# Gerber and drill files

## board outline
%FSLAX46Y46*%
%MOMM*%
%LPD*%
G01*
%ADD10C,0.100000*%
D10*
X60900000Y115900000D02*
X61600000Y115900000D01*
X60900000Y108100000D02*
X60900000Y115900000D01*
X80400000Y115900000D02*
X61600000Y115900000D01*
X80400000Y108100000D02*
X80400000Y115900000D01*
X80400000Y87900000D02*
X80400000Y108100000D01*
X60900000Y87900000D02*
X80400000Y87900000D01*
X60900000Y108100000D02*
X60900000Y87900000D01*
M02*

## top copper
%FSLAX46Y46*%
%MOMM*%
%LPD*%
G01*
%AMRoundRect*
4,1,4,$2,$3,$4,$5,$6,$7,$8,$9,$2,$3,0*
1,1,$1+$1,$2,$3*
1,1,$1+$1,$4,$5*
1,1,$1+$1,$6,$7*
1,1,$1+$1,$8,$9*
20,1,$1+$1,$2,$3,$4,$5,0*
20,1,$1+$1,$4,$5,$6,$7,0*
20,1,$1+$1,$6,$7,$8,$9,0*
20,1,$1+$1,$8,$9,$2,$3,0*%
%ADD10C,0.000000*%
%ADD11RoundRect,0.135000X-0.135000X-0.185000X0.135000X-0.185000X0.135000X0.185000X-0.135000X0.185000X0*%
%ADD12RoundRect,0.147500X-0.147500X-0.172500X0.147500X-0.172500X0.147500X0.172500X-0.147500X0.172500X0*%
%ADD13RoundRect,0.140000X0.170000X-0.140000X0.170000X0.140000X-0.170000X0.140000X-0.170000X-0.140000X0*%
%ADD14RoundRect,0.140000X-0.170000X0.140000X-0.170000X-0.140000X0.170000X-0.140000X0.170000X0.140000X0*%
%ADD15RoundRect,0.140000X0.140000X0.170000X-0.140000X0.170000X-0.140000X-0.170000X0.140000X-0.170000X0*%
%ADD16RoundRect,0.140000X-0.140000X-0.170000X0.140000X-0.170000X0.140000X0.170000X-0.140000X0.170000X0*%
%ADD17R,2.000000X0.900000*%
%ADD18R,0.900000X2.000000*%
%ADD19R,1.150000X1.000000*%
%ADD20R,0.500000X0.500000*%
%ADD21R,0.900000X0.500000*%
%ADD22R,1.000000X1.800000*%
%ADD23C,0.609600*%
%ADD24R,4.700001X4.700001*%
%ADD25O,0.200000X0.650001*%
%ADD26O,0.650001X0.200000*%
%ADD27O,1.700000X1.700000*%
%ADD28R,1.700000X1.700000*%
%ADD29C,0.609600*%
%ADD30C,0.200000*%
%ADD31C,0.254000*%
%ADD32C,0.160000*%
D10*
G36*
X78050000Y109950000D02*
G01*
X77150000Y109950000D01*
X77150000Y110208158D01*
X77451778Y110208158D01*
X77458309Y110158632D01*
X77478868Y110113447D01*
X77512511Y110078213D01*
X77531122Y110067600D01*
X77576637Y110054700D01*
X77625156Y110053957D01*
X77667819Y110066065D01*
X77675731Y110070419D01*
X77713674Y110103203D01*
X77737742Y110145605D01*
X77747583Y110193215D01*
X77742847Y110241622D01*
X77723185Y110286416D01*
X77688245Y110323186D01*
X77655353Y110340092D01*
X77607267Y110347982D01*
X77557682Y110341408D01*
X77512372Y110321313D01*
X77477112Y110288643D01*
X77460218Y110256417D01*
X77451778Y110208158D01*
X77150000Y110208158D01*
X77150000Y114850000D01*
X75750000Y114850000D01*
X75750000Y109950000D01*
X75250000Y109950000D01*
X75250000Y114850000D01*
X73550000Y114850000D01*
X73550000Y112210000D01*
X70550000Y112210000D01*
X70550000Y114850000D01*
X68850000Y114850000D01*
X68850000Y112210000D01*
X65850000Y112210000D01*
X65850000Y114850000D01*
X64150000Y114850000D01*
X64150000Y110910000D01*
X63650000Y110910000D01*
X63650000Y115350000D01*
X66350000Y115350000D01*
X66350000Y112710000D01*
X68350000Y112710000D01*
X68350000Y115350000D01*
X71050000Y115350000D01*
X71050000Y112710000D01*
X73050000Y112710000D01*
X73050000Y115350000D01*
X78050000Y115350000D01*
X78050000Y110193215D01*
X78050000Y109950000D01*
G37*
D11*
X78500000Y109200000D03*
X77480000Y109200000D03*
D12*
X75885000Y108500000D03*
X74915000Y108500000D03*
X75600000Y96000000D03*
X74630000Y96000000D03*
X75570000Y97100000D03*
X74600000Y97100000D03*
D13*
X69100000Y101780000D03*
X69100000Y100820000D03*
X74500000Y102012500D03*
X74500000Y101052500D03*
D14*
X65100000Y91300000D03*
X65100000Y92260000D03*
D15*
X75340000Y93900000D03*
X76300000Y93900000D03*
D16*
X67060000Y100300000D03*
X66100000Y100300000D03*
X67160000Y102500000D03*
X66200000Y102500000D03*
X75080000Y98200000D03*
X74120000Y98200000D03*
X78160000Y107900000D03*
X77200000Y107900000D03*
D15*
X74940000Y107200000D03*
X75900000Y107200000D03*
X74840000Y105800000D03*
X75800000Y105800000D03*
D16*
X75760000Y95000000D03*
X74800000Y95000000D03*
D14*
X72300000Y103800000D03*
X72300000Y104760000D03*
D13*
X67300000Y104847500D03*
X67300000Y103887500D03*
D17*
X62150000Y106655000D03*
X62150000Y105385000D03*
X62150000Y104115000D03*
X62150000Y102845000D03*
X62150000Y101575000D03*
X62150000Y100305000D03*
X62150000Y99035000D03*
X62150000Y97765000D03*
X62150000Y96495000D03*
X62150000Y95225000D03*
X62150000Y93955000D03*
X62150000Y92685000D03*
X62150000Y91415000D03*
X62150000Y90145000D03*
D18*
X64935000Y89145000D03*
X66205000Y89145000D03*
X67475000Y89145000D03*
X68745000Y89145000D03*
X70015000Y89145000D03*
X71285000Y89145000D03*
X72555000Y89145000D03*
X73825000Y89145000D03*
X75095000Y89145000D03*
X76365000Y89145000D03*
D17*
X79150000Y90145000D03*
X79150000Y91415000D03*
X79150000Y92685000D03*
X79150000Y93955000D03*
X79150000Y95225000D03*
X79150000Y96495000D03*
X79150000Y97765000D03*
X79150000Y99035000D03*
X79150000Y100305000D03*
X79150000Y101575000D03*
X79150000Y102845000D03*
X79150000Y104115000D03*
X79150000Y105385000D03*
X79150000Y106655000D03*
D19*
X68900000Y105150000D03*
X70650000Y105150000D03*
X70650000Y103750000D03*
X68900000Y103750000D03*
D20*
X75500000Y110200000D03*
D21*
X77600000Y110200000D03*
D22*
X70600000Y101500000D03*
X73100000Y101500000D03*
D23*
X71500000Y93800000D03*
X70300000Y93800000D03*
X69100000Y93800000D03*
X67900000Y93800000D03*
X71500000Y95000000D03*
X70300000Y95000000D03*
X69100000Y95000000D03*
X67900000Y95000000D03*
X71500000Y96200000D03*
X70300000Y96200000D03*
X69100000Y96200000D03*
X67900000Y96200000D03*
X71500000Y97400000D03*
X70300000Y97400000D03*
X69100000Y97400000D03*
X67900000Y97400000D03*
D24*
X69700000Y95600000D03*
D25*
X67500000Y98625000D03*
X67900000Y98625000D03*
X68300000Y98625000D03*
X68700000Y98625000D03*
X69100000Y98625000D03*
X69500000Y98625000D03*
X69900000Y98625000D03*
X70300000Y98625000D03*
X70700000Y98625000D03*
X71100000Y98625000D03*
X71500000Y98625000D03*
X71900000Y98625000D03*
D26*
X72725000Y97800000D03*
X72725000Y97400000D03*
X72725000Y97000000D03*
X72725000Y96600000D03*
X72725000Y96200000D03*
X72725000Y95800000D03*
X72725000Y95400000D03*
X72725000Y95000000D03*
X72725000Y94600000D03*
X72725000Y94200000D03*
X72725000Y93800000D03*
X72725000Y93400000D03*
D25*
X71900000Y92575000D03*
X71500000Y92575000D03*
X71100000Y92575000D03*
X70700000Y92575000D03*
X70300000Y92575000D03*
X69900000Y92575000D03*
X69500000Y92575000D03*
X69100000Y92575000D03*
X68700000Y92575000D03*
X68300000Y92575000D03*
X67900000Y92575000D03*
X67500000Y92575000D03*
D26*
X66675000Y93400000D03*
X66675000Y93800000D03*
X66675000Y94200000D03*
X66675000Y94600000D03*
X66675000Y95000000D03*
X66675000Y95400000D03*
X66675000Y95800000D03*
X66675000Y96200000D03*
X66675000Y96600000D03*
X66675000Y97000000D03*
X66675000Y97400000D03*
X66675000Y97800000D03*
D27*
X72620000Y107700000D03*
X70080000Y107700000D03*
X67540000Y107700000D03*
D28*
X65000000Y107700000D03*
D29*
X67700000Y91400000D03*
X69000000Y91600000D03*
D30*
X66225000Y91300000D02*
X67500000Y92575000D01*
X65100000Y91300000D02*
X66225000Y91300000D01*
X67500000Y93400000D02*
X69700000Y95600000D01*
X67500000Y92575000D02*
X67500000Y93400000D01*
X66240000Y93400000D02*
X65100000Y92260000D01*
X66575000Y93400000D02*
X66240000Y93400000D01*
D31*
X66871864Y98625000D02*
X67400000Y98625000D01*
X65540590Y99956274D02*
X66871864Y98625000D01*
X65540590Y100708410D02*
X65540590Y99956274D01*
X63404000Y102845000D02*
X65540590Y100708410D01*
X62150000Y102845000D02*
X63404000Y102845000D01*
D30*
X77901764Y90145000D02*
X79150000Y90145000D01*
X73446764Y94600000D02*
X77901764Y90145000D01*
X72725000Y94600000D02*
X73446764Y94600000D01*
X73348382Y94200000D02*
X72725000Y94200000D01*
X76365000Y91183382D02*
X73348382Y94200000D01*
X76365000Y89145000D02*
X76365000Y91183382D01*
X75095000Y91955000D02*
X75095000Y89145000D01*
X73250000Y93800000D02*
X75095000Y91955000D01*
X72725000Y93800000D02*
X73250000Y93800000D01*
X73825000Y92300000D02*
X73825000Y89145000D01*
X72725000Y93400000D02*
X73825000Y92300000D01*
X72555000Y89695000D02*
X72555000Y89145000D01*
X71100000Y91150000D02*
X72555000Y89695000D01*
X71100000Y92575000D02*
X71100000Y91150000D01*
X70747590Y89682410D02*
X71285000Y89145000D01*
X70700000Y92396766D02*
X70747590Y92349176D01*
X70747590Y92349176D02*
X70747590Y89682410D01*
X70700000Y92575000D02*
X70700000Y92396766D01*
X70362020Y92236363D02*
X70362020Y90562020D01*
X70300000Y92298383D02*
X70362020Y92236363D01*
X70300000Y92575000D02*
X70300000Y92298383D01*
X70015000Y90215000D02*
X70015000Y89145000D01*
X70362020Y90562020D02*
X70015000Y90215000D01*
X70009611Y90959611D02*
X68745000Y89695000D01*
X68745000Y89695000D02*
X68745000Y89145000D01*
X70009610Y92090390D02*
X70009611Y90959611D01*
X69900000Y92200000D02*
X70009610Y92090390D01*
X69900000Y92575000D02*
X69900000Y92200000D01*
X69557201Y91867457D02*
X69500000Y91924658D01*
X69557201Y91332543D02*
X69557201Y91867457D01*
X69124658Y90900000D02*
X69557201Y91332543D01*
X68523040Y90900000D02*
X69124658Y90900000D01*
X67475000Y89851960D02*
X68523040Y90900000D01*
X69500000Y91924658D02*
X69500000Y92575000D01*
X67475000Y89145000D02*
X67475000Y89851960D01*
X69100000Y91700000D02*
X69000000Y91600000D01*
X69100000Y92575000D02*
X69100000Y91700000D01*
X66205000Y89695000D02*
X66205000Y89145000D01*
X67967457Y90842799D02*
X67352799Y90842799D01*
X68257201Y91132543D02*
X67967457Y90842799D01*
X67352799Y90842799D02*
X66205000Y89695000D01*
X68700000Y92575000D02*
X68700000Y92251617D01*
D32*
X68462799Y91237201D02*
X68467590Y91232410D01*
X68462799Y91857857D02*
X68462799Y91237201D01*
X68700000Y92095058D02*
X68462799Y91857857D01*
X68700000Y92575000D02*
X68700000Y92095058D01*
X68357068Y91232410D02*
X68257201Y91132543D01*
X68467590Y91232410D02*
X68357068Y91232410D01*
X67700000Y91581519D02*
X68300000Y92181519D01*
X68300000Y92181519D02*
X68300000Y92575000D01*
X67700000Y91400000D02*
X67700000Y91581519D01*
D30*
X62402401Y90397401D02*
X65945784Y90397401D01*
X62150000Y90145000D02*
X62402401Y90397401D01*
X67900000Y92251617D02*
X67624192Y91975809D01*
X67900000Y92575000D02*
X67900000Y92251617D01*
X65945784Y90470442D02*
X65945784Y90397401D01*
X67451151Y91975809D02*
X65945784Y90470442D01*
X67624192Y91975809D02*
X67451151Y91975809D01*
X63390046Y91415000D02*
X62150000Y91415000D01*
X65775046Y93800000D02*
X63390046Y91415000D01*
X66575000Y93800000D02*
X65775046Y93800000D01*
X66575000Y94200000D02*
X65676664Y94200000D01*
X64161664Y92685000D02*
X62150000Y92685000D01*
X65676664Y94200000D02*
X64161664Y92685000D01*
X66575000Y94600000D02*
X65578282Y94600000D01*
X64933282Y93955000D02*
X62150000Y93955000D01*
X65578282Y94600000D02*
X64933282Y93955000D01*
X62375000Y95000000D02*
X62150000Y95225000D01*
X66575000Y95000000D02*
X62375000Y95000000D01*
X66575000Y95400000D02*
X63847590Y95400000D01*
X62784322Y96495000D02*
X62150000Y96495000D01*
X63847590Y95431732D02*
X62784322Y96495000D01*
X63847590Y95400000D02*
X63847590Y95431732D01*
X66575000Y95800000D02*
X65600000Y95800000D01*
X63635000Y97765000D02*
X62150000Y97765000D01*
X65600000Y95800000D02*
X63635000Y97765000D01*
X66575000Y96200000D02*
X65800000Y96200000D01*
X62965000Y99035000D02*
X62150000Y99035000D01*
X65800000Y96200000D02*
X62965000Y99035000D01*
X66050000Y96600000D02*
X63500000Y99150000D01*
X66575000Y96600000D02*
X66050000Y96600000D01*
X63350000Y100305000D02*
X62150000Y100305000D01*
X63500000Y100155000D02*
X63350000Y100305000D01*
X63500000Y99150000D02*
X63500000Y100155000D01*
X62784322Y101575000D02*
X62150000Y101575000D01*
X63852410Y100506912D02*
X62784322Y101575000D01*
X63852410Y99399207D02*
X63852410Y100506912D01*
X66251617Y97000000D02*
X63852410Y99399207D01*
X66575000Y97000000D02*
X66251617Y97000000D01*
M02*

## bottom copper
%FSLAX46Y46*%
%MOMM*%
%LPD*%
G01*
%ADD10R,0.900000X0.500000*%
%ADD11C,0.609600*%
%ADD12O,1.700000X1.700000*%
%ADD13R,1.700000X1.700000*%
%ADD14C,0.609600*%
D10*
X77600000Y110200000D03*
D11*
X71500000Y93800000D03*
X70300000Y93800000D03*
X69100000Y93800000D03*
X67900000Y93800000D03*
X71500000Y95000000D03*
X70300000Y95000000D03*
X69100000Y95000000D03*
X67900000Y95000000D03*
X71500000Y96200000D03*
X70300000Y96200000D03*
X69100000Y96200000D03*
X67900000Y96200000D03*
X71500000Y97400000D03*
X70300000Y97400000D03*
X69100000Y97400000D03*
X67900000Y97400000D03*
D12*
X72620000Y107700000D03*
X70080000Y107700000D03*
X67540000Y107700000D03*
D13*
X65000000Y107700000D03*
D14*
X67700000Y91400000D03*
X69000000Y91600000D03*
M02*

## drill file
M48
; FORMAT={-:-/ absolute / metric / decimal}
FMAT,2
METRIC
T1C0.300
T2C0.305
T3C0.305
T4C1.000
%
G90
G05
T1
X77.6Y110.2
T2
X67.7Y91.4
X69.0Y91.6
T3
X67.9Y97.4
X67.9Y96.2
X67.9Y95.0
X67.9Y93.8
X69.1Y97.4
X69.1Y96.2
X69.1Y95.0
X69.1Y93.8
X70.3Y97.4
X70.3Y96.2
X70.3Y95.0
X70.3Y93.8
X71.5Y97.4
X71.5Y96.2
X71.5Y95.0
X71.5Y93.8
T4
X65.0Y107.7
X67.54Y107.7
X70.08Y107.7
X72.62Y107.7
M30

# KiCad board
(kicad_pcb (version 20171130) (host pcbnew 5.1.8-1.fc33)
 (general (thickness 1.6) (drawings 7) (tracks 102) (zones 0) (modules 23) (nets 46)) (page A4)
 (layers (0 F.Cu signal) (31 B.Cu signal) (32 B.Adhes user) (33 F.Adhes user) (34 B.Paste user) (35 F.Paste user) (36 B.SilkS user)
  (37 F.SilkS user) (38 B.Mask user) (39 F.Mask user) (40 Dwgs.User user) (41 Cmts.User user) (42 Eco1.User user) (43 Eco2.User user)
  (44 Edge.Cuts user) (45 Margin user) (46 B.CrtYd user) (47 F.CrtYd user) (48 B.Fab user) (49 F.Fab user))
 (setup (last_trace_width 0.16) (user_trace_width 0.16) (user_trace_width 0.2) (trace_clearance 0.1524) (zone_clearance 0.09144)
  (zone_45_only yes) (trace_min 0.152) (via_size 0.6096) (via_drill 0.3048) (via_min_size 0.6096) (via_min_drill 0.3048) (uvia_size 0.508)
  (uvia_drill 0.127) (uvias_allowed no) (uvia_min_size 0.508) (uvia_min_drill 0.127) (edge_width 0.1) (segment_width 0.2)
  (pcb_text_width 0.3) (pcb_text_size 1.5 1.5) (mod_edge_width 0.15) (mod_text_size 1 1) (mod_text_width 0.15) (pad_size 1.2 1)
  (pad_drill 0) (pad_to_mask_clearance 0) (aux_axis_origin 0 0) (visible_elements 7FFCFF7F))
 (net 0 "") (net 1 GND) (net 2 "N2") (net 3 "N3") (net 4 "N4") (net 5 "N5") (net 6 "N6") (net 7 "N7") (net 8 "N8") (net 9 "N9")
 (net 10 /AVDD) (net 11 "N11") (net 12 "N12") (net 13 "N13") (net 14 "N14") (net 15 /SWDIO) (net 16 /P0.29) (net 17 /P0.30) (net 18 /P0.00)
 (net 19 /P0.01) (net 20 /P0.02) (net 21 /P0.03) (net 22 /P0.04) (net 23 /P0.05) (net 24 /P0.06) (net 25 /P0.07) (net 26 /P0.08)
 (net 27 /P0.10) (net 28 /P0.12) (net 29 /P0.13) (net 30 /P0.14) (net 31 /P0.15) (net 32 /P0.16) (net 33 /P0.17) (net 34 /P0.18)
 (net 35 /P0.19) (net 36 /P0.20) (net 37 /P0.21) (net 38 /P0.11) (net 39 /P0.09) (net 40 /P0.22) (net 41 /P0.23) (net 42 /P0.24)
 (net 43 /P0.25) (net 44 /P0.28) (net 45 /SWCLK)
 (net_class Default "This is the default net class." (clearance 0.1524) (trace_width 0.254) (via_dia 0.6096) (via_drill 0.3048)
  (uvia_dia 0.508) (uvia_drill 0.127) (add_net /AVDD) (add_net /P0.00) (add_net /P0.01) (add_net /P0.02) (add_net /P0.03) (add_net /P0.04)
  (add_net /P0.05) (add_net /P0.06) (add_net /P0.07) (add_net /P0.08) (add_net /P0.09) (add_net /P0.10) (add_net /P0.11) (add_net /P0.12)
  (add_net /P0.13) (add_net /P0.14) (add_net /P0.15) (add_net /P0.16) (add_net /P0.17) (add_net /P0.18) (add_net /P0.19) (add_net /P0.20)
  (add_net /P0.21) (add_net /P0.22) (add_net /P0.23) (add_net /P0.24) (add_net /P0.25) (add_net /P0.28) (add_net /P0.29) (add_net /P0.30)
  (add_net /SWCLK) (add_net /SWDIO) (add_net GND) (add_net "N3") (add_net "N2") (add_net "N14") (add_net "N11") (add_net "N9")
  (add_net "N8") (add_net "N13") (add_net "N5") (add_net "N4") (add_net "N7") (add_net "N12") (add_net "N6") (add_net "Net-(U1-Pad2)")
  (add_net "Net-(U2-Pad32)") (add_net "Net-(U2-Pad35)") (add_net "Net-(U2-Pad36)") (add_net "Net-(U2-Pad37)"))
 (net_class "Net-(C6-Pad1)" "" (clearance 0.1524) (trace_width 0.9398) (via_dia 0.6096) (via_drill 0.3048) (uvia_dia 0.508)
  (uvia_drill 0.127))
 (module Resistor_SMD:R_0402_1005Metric (layer F.Cu) (at 77.99 -109.2)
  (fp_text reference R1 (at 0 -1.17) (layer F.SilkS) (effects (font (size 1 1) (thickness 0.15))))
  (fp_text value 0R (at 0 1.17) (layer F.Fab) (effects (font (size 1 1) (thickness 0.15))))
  (pad 2 smd roundrect (at 0.51 0) (size 0.54 0.64) (layers F.Cu F.Paste F.Mask) (roundrect_rratio 0.25) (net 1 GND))
  (pad 1 smd roundrect (at -0.51 0) (size 0.54 0.64) (layers F.Cu F.Paste F.Mask) (roundrect_rratio 0.25) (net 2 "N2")))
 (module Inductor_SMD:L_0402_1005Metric (layer F.Cu) (at 75.4 -108.5)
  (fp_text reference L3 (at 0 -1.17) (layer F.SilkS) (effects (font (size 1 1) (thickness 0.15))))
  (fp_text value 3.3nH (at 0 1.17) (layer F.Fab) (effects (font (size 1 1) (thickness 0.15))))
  (pad 2 smd roundrect (at 0.485 0) (size 0.59 0.64) (layers F.Cu F.Paste F.Mask) (roundrect_rratio 0.25) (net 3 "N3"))
  (pad 1 smd roundrect (at -0.485 0) (size 0.59 0.64) (layers F.Cu F.Paste F.Mask) (roundrect_rratio 0.25) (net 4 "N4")))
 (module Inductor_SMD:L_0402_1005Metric (layer F.Cu) (at 75.115 -96)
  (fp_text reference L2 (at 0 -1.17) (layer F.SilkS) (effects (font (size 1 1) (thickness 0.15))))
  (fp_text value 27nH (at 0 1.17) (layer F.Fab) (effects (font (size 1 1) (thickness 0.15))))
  (pad 2 smd roundrect (at 0.485 0) (size 0.59 0.64) (layers F.Cu F.Paste F.Mask) (roundrect_rratio 0.25) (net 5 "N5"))
  (pad 1 smd roundrect (at -0.485 0) (size 0.59 0.64) (layers F.Cu F.Paste F.Mask) (roundrect_rratio 0.25) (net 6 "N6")))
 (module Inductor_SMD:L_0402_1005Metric (layer F.Cu) (at 75.085 -97.1)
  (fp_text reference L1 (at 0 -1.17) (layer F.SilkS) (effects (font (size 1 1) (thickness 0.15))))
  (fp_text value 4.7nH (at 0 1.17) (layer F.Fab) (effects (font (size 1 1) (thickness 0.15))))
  (pad 2 smd roundrect (at 0.485 0) (size 0.59 0.64) (layers F.Cu F.Paste F.Mask) (roundrect_rratio 0.25) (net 6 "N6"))
  (pad 1 smd roundrect (at -0.485 0) (size 0.59 0.64) (layers F.Cu F.Paste F.Mask) (roundrect_rratio 0.25) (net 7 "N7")))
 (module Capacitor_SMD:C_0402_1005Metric (layer F.Cu) (at 69.1 -101.3 90)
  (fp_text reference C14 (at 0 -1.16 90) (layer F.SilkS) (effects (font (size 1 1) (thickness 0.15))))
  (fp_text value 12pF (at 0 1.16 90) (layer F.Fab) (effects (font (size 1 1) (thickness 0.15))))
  (pad 2 smd roundrect (at 0.48 0 90) (size 0.56 0.62) (layers F.Cu F.Paste F.Mask) (roundrect_rratio 0.25) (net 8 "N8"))
  (pad 1 smd roundrect (at -0.48 0 90) (size 0.56 0.62) (layers F.Cu F.Paste F.Mask) (roundrect_rratio 0.25) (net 1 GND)))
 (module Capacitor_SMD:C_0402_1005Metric (layer F.Cu) (at 74.5 -101.5325 90)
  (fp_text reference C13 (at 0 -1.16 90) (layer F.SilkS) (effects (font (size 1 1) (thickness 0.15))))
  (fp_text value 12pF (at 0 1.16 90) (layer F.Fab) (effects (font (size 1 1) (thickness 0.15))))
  (pad 2 smd roundrect (at 0.48 0 90) (size 0.56 0.62) (layers F.Cu F.Paste F.Mask) (roundrect_rratio 0.25) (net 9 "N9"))
  (pad 1 smd roundrect (at -0.48 0 90) (size 0.56 0.62) (layers F.Cu F.Paste F.Mask) (roundrect_rratio 0.25) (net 1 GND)))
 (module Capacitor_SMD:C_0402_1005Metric (layer F.Cu) (at 65.1 -91.78 270)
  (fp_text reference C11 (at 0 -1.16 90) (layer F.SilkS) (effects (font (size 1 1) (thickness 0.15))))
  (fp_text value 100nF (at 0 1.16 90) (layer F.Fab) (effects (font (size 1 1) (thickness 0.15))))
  (pad 2 smd roundrect (at 0.48 0 270) (size 0.56 0.62) (layers F.Cu F.Paste F.Mask) (roundrect_rratio 0.25) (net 1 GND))
  (pad 1 smd roundrect (at -0.48 0 270) (size 0.56 0.62) (layers F.Cu F.Paste F.Mask) (roundrect_rratio 0.25) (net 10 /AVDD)))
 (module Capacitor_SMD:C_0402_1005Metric (layer F.Cu) (at 75.82 -93.9 180)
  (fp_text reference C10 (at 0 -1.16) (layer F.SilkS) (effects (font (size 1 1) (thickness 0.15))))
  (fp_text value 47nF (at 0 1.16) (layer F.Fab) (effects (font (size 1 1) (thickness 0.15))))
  (pad 2 smd roundrect (at 0.48 0 180) (size 0.56 0.62) (layers F.Cu F.Paste F.Mask) (roundrect_rratio 0.25) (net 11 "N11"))
  (pad 1 smd roundrect (at -0.48 0 180) (size 0.56 0.62) (layers F.Cu F.Paste F.Mask) (roundrect_rratio 0.25) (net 1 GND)))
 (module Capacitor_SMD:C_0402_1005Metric (layer F.Cu) (at 66.58 -100.3)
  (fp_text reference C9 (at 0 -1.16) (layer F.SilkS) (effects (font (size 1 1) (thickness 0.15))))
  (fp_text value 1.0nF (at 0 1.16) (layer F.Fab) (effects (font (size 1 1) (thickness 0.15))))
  (pad 2 smd roundrect (at 0.48 0) (size 0.56 0.62) (layers F.Cu F.Paste F.Mask) (roundrect_rratio 0.25) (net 1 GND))
  (pad 1 smd roundrect (at -0.48 0) (size 0.56 0.62) (layers F.Cu F.Paste F.Mask) (roundrect_rratio 0.25) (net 10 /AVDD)))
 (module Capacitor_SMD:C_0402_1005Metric (layer F.Cu) (at 66.68 -102.5)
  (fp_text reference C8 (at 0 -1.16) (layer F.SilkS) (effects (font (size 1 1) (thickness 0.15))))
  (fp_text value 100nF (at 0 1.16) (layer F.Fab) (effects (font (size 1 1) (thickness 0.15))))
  (pad 2 smd roundrect (at 0.48 0) (size 0.56 0.62) (layers F.Cu F.Paste F.Mask) (roundrect_rratio 0.25) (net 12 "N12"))
  (pad 1 smd roundrect (at -0.48 0) (size 0.56 0.62) (layers F.Cu F.Paste F.Mask) (roundrect_rratio 0.25) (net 1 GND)))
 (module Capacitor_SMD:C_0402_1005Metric (layer F.Cu) (at 74.6 -98.2)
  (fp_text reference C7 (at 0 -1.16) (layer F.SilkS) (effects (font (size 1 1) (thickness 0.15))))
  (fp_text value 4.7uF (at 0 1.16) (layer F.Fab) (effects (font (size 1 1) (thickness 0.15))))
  (pad 2 smd roundrect (at 0.48 0) (size 0.56 0.62) (layers F.Cu F.Paste F.Mask) (roundrect_rratio 0.25) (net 1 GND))
  (pad 1 smd roundrect (at -0.48 0) (size 0.56 0.62) (layers F.Cu F.Paste F.Mask) (roundrect_rratio 0.25) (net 10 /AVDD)))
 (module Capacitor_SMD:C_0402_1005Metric (layer F.Cu) (at 77.68 -107.9)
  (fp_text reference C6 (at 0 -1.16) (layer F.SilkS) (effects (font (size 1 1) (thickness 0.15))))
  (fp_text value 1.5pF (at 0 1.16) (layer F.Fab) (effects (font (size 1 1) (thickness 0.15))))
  (pad 2 smd roundrect (at 0.48 0) (size 0.56 0.62) (layers F.Cu F.Paste F.Mask) (roundrect_rratio 0.25) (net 1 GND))
  (pad 1 smd roundrect (at -0.48 0) (size 0.56 0.62) (layers F.Cu F.Paste F.Mask) (roundrect_rratio 0.25) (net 3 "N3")))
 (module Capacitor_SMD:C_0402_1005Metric (layer F.Cu) (at 75.42 -107.2 180)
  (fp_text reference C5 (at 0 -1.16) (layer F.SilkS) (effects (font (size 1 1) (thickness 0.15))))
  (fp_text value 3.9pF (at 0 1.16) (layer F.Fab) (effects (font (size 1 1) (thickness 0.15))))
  (pad 2 smd roundrect (at 0.48 0 180) (size 0.56 0.62) (layers F.Cu F.Paste F.Mask) (roundrect_rratio 0.25) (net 7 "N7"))
  (pad 1 smd roundrect (at -0.48 0 180) (size 0.56 0.62) (layers F.Cu F.Paste F.Mask) (roundrect_rratio 0.25) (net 4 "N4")))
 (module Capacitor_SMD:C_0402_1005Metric (layer F.Cu) (at 75.32 -105.8 180)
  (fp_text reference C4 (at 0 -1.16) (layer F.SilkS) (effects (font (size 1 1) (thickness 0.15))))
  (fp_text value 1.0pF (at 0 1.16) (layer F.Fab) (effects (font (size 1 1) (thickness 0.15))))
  (pad 2 smd roundrect (at 0.48 0 180) (size 0.56 0.62) (layers F.Cu F.Paste F.Mask) (roundrect_rratio 0.25) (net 1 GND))
  (pad 1 smd roundrect (at -0.48 0 180) (size 0.56 0.62) (layers F.Cu F.Paste F.Mask) (roundrect_rratio 0.25) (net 4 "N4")))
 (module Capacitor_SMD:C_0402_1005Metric (layer F.Cu) (at 75.28 -95)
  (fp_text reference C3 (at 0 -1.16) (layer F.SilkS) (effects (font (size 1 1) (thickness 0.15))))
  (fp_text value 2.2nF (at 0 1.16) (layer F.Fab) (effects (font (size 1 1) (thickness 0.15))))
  (pad 2 smd roundrect (at 0.48 0) (size 0.56 0.62) (layers F.Cu F.Paste F.Mask) (roundrect_rratio 0.25) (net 1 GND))
  (pad 1 smd roundrect (at -0.48 0) (size 0.56 0.62) (layers F.Cu F.Paste F.Mask) (roundrect_rratio 0.25) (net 5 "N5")))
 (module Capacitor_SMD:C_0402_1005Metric (layer F.Cu) (at 72.3 -104.28 270)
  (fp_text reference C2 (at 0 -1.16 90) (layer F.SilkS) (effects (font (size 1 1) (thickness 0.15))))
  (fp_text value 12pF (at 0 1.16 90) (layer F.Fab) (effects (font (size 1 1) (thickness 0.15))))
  (pad 2 smd roundrect (at 0.48 0 270) (size 0.56 0.62) (layers F.Cu F.Paste F.Mask) (roundrect_rratio 0.25) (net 1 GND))
  (pad 1 smd roundrect (at -0.48 0 270) (size 0.56 0.62) (layers F.Cu F.Paste F.Mask) (roundrect_rratio 0.25) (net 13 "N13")))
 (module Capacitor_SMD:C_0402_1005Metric (layer F.Cu) (at 67.3 -104.3675 90)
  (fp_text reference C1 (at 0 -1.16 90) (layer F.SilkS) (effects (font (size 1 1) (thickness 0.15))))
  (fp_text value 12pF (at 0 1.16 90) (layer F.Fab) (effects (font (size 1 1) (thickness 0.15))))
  (pad 2 smd roundrect (at 0.48 0 90) (size 0.56 0.62) (layers F.Cu F.Paste F.Mask) (roundrect_rratio 0.25) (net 1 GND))
  (pad 1 smd roundrect (at -0.48 0 90) (size 0.56 0.62) (layers F.Cu F.Paste F.Mask) (roundrect_rratio 0.25) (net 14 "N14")))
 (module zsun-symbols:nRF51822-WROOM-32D (layer F.Cu) (at 70.65 -98.4)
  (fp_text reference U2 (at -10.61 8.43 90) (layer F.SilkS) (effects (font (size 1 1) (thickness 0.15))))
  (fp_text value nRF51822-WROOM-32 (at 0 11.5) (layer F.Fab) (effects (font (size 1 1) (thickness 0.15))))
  (pad 1 smd rect (at -8.5 -8.255) (size 2 0.9) (layers F.Cu F.Paste F.Mask) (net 1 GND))
  (pad 2 smd rect (at -8.5 -6.985) (size 2 0.9) (layers F.Cu F.Paste F.Mask) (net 10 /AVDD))
  (pad 3 smd rect (at -8.5 -5.715) (size 2 0.9) (layers F.Cu F.Paste F.Mask) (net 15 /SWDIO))
  (pad 4 smd rect (at -8.5 -4.445) (size 2 0.9) (layers F.Cu F.Paste F.Mask) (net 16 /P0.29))
  (pad 5 smd rect (at -8.5 -3.175) (size 2 0.9) (layers F.Cu F.Paste F.Mask) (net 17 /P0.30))
  (pad 6 smd rect (at -8.5 -1.905) (size 2 0.9) (layers F.Cu F.Paste F.Mask) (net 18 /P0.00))
  (pad 7 smd rect (at -8.5 -0.635) (size 2 0.9) (layers F.Cu F.Paste F.Mask) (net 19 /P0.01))
  (pad 8 smd rect (at -8.5 0.635) (size 2 0.9) (layers F.Cu F.Paste F.Mask) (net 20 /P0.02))
  (pad 9 smd rect (at -8.5 1.905) (size 2 0.9) (layers F.Cu F.Paste F.Mask) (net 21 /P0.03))
  (pad 10 smd rect (at -8.5 3.175) (size 2 0.9) (layers F.Cu F.Paste F.Mask) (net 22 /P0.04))
  (pad 11 smd rect (at -8.5 4.445) (size 2 0.9) (layers F.Cu F.Paste F.Mask) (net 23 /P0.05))
  (pad 12 smd rect (at -8.5 5.715) (size 2 0.9) (layers F.Cu F.Paste F.Mask) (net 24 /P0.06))
  (pad 13 smd rect (at -8.5 6.985) (size 2 0.9) (layers F.Cu F.Paste F.Mask) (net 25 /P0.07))
  (pad 14 smd rect (at -8.5 8.255) (size 2 0.9) (layers F.Cu F.Paste F.Mask) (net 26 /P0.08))
  (pad 15 smd rect (at -5.715 9.255 90) (size 2 0.9) (layers F.Cu F.Paste F.Mask) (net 1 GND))
  (pad 16 smd rect (at -4.445 9.255 90) (size 2 0.9) (layers F.Cu F.Paste F.Mask) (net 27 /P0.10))
  (pad 17 smd rect (at -3.175 9.255 90) (size 2 0.9) (layers F.Cu F.Paste F.Mask) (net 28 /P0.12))
  (pad 18 smd rect (at -1.905 9.255 90) (size 2 0.9) (layers F.Cu F.Paste F.Mask) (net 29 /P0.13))
  (pad 19 smd rect (at -0.635 9.255 90) (size 2 0.9) (layers F.Cu F.Paste F.Mask) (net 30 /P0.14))
  (pad 20 smd rect (at 0.635 9.255 90) (size 2 0.9) (layers F.Cu F.Paste F.Mask) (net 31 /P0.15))
  (pad 21 smd rect (at 1.905 9.255 90) (size 2 0.9) (layers F.Cu F.Paste F.Mask) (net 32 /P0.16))
  (pad 22 smd rect (at 3.175 9.255 90) (size 2 0.9) (layers F.Cu F.Paste F.Mask) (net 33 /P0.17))
  (pad 23 smd rect (at 4.445 9.255 90) (size 2 0.9) (layers F.Cu F.Paste F.Mask) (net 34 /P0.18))
  (pad 24 smd rect (at 5.715 9.255 90) (size 2 0.9) (layers F.Cu F.Paste F.Mask) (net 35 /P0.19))
  (pad 25 smd rect (at 8.5 8.255) (size 2 0.9) (layers F.Cu F.Paste F.Mask) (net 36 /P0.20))
  (pad 26 smd rect (at 8.5 6.985) (size 2 0.9) (layers F.Cu F.Paste F.Mask) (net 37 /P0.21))
  (pad 27 smd rect (at 8.5 5.715) (size 2 0.9) (layers F.Cu F.Paste F.Mask) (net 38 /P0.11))
  (pad 28 smd rect (at 8.5 4.445) (size 2 0.9) (layers F.Cu F.Paste F.Mask) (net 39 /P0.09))
  (pad 29 smd rect (at 8.5 3.175) (size 2 0.9) (layers F.Cu F.Paste F.Mask) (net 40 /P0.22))
  (pad 30 smd rect (at 8.5 1.905) (size 2 0.9) (layers F.Cu F.Paste F.Mask) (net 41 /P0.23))
  (pad 31 smd rect (at 8.5 0.635) (size 2 0.9) (layers F.Cu F.Paste F.Mask) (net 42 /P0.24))
  (pad 32 smd rect (at 8.5 -0.635) (size 2 0.9) (layers F.Cu F.Paste F.Mask))
  (pad 33 smd rect (at 8.5 -1.905) (size 2 0.9) (layers F.Cu F.Paste F.Mask) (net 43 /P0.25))
  (pad 34 smd rect (at 8.5 -3.175) (size 2 0.9) (layers F.Cu F.Paste F.Mask) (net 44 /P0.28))
  (pad 35 smd rect (at 8.5 -4.445) (size 2 0.9) (layers F.Cu F.Paste F.Mask))
  (pad 36 smd rect (at 8.5 -5.715) (size 2 0.9) (layers F.Cu F.Paste F.Mask))
  (pad 37 smd rect (at 8.5 -6.985) (size 2 0.9) (layers F.Cu F.Paste F.Mask))
  (pad 38 smd rect (at 8.5 -8.255) (size 2 0.9) (layers F.Cu F.Paste F.Mask) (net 1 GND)))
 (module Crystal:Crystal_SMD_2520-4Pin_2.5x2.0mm (layer F.Cu) (at 69.775 -104.45)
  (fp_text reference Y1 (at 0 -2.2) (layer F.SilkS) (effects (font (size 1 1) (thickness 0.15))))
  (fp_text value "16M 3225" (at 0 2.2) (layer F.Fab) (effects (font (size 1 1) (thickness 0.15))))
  (pad 4 smd rect (at -0.875 -0.7) (size 1.15 1) (layers F.Cu F.Paste F.Mask) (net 1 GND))
  (pad 3 smd rect (at 0.875 -0.7) (size 1.15 1) (layers F.Cu F.Paste F.Mask) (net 13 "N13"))
  (pad 2 smd rect (at 0.875 0.7) (size 1.15 1) (layers F.Cu F.Paste F.Mask) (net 1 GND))
  (pad 1 smd rect (at -0.875 0.7) (size 1.15 1) (layers F.Cu F.Paste F.Mask) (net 14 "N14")))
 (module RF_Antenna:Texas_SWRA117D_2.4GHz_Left (layer F.Cu) (at 75.5 -110.2)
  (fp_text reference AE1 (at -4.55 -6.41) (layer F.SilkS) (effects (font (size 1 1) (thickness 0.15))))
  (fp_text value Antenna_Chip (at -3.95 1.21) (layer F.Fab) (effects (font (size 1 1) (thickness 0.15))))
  (fp_poly
   (pts (xy -2.45 -2.51) (xy -4.45 -2.51) (xy -4.45 -5.15) (xy -7.15 -5.15) (xy -7.15 -2.51) (xy -9.15 -2.51) (xy -9.15 -5.15)
    (xy -11.85 -5.15) (xy -11.85 -0.71) (xy -11.35 -0.71) (xy -11.35 -4.65) (xy -9.65 -4.65) (xy -9.65 -2.01) (xy -6.65 -2.01)
    (xy -6.65 -4.65) (xy -4.95 -4.65) (xy -4.95 -2.01) (xy -1.95 -2.01) (xy -1.95 -4.65) (xy -0.25 -4.65) (xy -0.25 0.25) (xy 0.25 0.25)
    (xy 0.25 -4.65) (xy 1.65 -4.65) (xy 1.65 0.25) (xy 2.55 0.25) (xy 2.55 0.006785) (xy 2.247583 0.006785) (xy 2.237742 0.054395)
    (xy 2.213674 0.096797) (xy 2.175731 0.129581) (xy 2.167819 0.133935) (xy 2.125156 0.146043) (xy 2.076637 0.1453) (xy 2.031122 0.1324)
    (xy 2.012511 0.121787) (xy 1.978868 0.086553) (xy 1.958309 0.041368) (xy 1.951778 -0.008158) (xy 1.960218 -0.056417)
    (xy 1.977112 -0.088643) (xy 2.012372 -0.121313) (xy 2.057682 -0.141408) (xy 2.107267 -0.147982) (xy 2.155353 -0.140092)
    (xy 2.188245 -0.123186) (xy 2.223185 -0.086416) (xy 2.242847 -0.041622) (xy 2.247583 0.006785) (xy 2.55 0.006785) (xy 2.55 -5.15)
    (xy -2.45 -5.15) (xy -2.45 -2.51))
   (layer F.Cu) (width 0))
  (pad 1 connect rect (at 0 0) (size 0.5 0.5) (layers F.Cu) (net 3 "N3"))
  (pad 2 thru_hole rect (at 2.1 0) (size 0.9 0.5) (drill 0.3) (layers *.Cu) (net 2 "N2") (zone_connect 2)))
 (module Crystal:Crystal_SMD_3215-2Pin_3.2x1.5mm (layer F.Cu) (at 71.85 -101.5)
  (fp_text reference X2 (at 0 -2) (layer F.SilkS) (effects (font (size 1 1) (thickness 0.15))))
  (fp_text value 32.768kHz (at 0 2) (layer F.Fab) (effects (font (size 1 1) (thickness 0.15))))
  (pad 2 smd rect (at -1.25 0) (size 1 1.8) (layers F.Cu F.Paste F.Mask) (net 8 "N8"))
  (pad 1 smd rect (at 1.25 0) (size 1 1.8) (layers F.Cu F.Paste F.Mask) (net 9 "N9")))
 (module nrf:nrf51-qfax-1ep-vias (layer F.Cu) (at 69.7 -95.6)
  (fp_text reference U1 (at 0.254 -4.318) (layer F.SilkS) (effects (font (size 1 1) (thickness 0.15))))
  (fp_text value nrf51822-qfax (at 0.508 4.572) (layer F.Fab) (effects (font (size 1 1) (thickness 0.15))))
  (pad 49 thru_hole circle (at 1.8 1.8) (size 0.6096 0.6096) (drill 0.3048) (layers *.Cu *.Mask F.SilkS) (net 1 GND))
  (pad 49 thru_hole circle (at 0.6 1.8) (size 0.6096 0.6096) (drill 0.3048) (layers *.Cu *.Mask F.SilkS) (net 1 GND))
  (pad 49 thru_hole circle (at -0.6 1.8) (size 0.6096 0.6096) (drill 0.3048) (layers *.Cu *.Mask F.SilkS) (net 1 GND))
  (pad 49 thru_hole circle (at -1.8 1.8) (size 0.6096 0.6096) (drill 0.3048) (layers *.Cu *.Mask F.SilkS) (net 1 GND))
  (pad 49 thru_hole circle (at 1.8 0.6) (size 0.6096 0.6096) (drill 0.3048) (layers *.Cu *.Mask F.SilkS) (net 1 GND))
  (pad 49 thru_hole circle (at 0.6 0.6) (size 0.6096 0.6096) (drill 0.3048) (layers *.Cu *.Mask F.SilkS) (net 1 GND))
  (pad 49 thru_hole circle (at -0.6 0.6) (size 0.6096 0.6096) (drill 0.3048) (layers *.Cu *.Mask F.SilkS) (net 1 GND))
  (pad 49 thru_hole circle (at -1.8 0.6) (size 0.6096 0.6096) (drill 0.3048) (layers *.Cu *.Mask F.SilkS) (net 1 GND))
  (pad 49 thru_hole circle (at 1.8 -0.6) (size 0.6096 0.6096) (drill 0.3048) (layers *.Cu *.Mask F.SilkS) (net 1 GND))
  (pad 49 thru_hole circle (at 0.6 -0.6) (size 0.6096 0.6096) (drill 0.3048) (layers *.Cu *.Mask F.SilkS) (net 1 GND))
  (pad 49 thru_hole circle (at -0.6 -0.6) (size 0.6096 0.6096) (drill 0.3048) (layers *.Cu *.Mask F.SilkS) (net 1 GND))
  (pad 49 thru_hole circle (at -1.8 -0.6) (size 0.6096 0.6096) (drill 0.3048) (layers *.Cu *.Mask F.SilkS) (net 1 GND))
  (pad 49 thru_hole circle (at 1.8 -1.8) (size 0.6096 0.6096) (drill 0.3048) (layers *.Cu *.Mask F.SilkS) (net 1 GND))
  (pad 49 thru_hole circle (at 0.6 -1.8) (size 0.6096 0.6096) (drill 0.3048) (layers *.Cu *.Mask F.SilkS) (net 1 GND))
  (pad 49 thru_hole circle (at -0.6 -1.8) (size 0.6096 0.6096) (drill 0.3048) (layers *.Cu *.Mask F.SilkS) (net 1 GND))
  (pad 49 thru_hole circle (at -1.8 -1.8) (size 0.6096 0.6096) (drill 0.3048) (layers *.Cu *.Mask F.SilkS) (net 1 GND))
  (pad 49 smd rect (at 0 0) (size 4.700001 4.700001) (layers F.Cu F.Paste F.Mask) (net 1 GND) (solder_paste_margin_ratio -0.2))
  (pad 48 smd oval (at -2.2 -3.025) (size 0.2 0.650001) (layers F.Cu F.Paste F.Mask) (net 16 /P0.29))
  (pad 47 smd oval (at -1.8 -3.025) (size 0.2 0.650001) (layers F.Cu F.Paste F.Mask) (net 44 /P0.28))
  (pad 46 smd oval (at -1.4 -3.025) (size 0.2 0.650001) (layers F.Cu F.Paste F.Mask) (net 8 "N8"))
  (pad 45 smd oval (at -1 -3.025) (size 0.2 0.650001) (layers F.Cu F.Paste F.Mask) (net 9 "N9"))
  (pad 44 smd oval (at -0.6 -3.025) (size 0.2 0.650001) (layers F.Cu F.Paste F.Mask) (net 43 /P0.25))
  (pad 43 smd oval (at -0.2 -3.025) (size 0.2 0.650001) (layers F.Cu F.Paste F.Mask) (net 42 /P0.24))
  (pad 42 smd oval (at 0.2 -3.025) (size 0.2 0.650001) (layers F.Cu F.Paste F.Mask) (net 41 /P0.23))
  (pad 41 smd oval (at 0.6 -3.025) (size 0.2 0.650001) (layers F.Cu F.Paste F.Mask) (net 40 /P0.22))
  (pad 40 smd oval (at 1 -3.025) (size 0.2 0.650001) (layers F.Cu F.Paste F.Mask) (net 37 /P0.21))
  (pad 39 smd oval (at 1.4 -3.025) (size 0.2 0.650001) (layers F.Cu F.Paste F.Mask) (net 12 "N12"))
  (pad 38 smd oval (at 1.8 -3.025) (size 0.2 0.650001) (layers F.Cu F.Paste F.Mask) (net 13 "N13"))
  (pad 37 smd oval (at 2.2 -3.025) (size 0.2 0.650001) (layers F.Cu F.Paste F.Mask) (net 14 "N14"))
  (pad 36 smd oval (at 3.025 -2.2 90) (size 0.2 0.650001) (layers F.Cu F.Paste F.Mask) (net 10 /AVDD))
  (pad 35 smd oval (at 3.025 -1.8 90) (size 0.2 0.650001) (layers F.Cu F.Paste F.Mask) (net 10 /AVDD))
  (pad 34 smd oval (at 3.025 -1.4 90) (size 0.2 0.650001) (layers F.Cu F.Paste F.Mask) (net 1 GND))
  (pad 33 smd oval (at 3.025 -1 90) (size 0.2 0.650001) (layers F.Cu F.Paste F.Mask) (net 1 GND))
  (pad 32 smd oval (at 3.025 -0.6 90) (size 0.2 0.650001) (layers F.Cu F.Paste F.Mask) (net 7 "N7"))
  (pad 31 smd oval (at 3.025 -0.2 90) (size 0.2 0.650001) (layers F.Cu F.Paste F.Mask) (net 6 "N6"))
  (pad 30 smd oval (at 3.025 0.2 90) (size 0.2 0.650001) (layers F.Cu F.Paste F.Mask) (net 5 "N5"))
  (pad 29 smd oval (at 3.025 0.6 90) (size 0.2 0.650001) (layers F.Cu F.Paste F.Mask) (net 11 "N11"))
  (pad 28 smd oval (at 3.025 1 90) (size 0.2 0.650001) (layers F.Cu F.Paste F.Mask) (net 36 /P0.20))
  (pad 27 smd oval (at 3.025 1.4 90) (size 0.2 0.650001) (layers F.Cu F.Paste F.Mask) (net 35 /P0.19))
  (pad 26 smd oval (at 3.025 1.8 90) (size 0.2 0.650001) (layers F.Cu F.Paste F.Mask) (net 34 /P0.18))
  (pad 25 smd oval (at 3.025 2.2 90) (size 0.2 0.650001) (layers F.Cu F.Paste F.Mask) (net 33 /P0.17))
  (pad 24 smd oval (at 2.2 3.025) (size 0.2 0.650001) (layers F.Cu F.Paste F.Mask) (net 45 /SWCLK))
  (pad 23 smd oval (at 1.8 3.025) (size 0.2 0.650001) (layers F.Cu F.Paste F.Mask) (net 15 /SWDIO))
  (pad 22 smd oval (at 1.4 3.025) (size 0.2 0.650001) (layers F.Cu F.Paste F.Mask) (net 32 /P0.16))
  (pad 21 smd oval (at 1 3.025) (size 0.2 0.650001) (layers F.Cu F.Paste F.Mask) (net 31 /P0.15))
  (pad 20 smd oval (at 0.6 3.025) (size 0.2 0.650001) (layers F.Cu F.Paste F.Mask) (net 30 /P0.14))
  (pad 19 smd oval (at 0.2 3.025) (size 0.2 0.650001) (layers F.Cu F.Paste F.Mask) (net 29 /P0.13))
  (pad 18 smd oval (at -0.2 3.025) (size 0.2 0.650001) (layers F.Cu F.Paste F.Mask) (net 28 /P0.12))
  (pad 17 smd oval (at -0.6 3.025) (size 0.2 0.650001) (layers F.Cu F.Paste F.Mask) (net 38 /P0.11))
  (pad 16 smd oval (at -1 3.025) (size 0.2 0.650001) (layers F.Cu F.Paste F.Mask) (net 27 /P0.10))
  (pad 15 smd oval (at -1.4 3.025) (size 0.2 0.650001) (layers F.Cu F.Paste F.Mask) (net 39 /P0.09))
  (pad 14 smd oval (at -1.8 3.025) (size 0.2 0.650001) (layers F.Cu F.Paste F.Mask) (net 26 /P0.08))
  (pad 13 smd oval (at -2.2 3.025) (size 0.2 0.650001) (layers F.Cu F.Paste F.Mask) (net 1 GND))
  (pad 12 smd oval (at -3.025 2.2 90) (size 0.2 0.650001) (layers F.Cu F.Paste F.Mask) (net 10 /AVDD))
  (pad 11 smd oval (at -3.025 1.8 90) (size 0.2 0.650001) (layers F.Cu F.Paste F.Mask) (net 25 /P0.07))
  (pad 10 smd oval (at -3.025 1.4 90) (size 0.2 0.650001) (layers F.Cu F.Paste F.Mask) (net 24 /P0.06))
  (pad 9 smd oval (at -3.025 1 90) (size 0.2 0.650001) (layers F.Cu F.Paste F.Mask) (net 23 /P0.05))
  (pad 8 smd oval (at -3.025 0.6 90) (size 0.2 0.650001) (layers F.Cu F.Paste F.Mask) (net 22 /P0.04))
  (pad 7 smd oval (at -3.025 0.2 90) (size 0.2 0.650001) (layers F.Cu F.Paste F.Mask) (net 21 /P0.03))
  (pad 6 smd oval (at -3.025 -0.2 90) (size 0.2 0.650001) (layers F.Cu F.Paste F.Mask) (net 20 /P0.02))
  (pad 5 smd oval (at -3.025 -0.6 90) (size 0.2 0.650001) (layers F.Cu F.Paste F.Mask) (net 19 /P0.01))
  (pad 4 smd oval (at -3.025 -1 90) (size 0.2 0.650001) (layers F.Cu F.Paste F.Mask) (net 18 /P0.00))
  (pad 3 smd oval (at -3.025 -1.4 90) (size 0.2 0.650001) (layers F.Cu F.Paste F.Mask) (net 17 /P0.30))
  (pad 2 smd oval (at -3.025 -1.8 90) (size 0.2 0.650001) (layers F.Cu F.Paste F.Mask))
  (pad 1 smd oval (at -3.025 -2.2 90) (size 0.2 0.650001) (layers F.Cu F.Paste F.Mask) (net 10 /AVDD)))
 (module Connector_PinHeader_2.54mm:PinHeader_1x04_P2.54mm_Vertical (layer F.Cu) (at 65 -107.7 90)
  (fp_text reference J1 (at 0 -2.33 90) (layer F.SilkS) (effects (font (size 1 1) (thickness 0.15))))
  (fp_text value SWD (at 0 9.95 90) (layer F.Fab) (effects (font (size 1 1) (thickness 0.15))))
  (pad 4 thru_hole oval (at 0 7.62 90) (size 1.7 1.7) (drill 1) (layers *.Cu *.Mask) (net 10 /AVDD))
  (pad 3 thru_hole oval (at 0 5.08 90) (size 1.7 1.7) (drill 1) (layers *.Cu *.Mask) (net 1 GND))
  (pad 2 thru_hole oval (at 0 2.54 90) (size 1.7 1.7) (drill 1) (layers *.Cu *.Mask) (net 15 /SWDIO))
  (pad 1 thru_hole rect (at 0 0 90) (size 1.7 1.7) (drill 1) (layers *.Cu *.Mask) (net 45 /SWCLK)))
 (gr_line (start 60.9 -115.9) (end 61.6 -115.9) (layer Edge.Cuts) (width 0.1))
 (gr_line (start 60.9 -108.1) (end 60.9 -115.9) (layer Edge.Cuts) (width 0.1))
 (gr_line (start 80.4 -115.9) (end 61.6 -115.9) (layer Edge.Cuts) (width 0.1))
 (gr_line (start 80.4 -108.1) (end 80.4 -115.9) (layer Edge.Cuts) (width 0.1))
 (gr_line (start 80.4 -87.9) (end 80.4 -108.1) (layer Edge.Cuts) (width 0.1))
 (gr_line (start 60.9 -87.9) (end 80.4 -87.9) (layer Edge.Cuts) (width 0.1))
 (gr_line (start 60.9 -108.1) (end 60.9 -87.9) (layer Edge.Cuts) (width 0.1))
 (via (at 67.7 -91.4) (size 0.6096) (drill 0.3048) (layers F.Cu B.Cu) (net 39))
 (via (at 69 -91.6) (size 0.6096) (drill 0.3048) (layers F.Cu B.Cu) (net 38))
 (segment (start 66.225 -91.3) (end 67.5 -92.575) (width 0.2) (layer F.Cu) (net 1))
 (segment (start 65.1 -91.3) (end 66.225 -91.3) (width 0.2) (layer F.Cu) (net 1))
 (segment (start 67.5 -93.4) (end 69.7 -95.6) (width 0.2) (layer F.Cu) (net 1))
 (segment (start 67.5 -92.575) (end 67.5 -93.4) (width 0.2) (layer F.Cu) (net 1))
 (segment (start 66.24 -93.4) (end 65.1 -92.26) (width 0.2) (layer F.Cu) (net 10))
 (segment (start 66.575 -93.4) (end 66.24 -93.4) (width 0.2) (layer F.Cu) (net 10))
 (segment (start 66.871864 -98.625) (end 67.4 -98.625) (width 0.254) (layer F.Cu) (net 16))
 (segment (start 65.54059 -99.956274) (end 66.871864 -98.625) (width 0.254) (layer F.Cu) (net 16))
 (segment (start 65.54059 -100.70841) (end 65.54059 -99.956274) (width 0.254) (layer F.Cu) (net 16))
 (segment (start 63.404 -102.845) (end 65.54059 -100.70841) (width 0.254) (layer F.Cu) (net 16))
 (segment (start 62.15 -102.845) (end 63.404 -102.845) (width 0.254) (layer F.Cu) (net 16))
 (segment (start 77.901764 -90.145) (end 79.15 -90.145) (width 0.2) (layer F.Cu) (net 36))
 (segment (start 73.446764 -94.6) (end 77.901764 -90.145) (width 0.2) (layer F.Cu) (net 36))
 (segment (start 72.725 -94.6) (end 73.446764 -94.6) (width 0.2) (layer F.Cu) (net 36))
 (segment (start 73.348382 -94.2) (end 72.725 -94.2) (width 0.2) (layer F.Cu) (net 35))
 (segment (start 76.365 -91.183382) (end 73.348382 -94.2) (width 0.2) (layer F.Cu) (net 35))
 (segment (start 76.365 -89.145) (end 76.365 -91.183382) (width 0.2) (layer F.Cu) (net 35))
 (segment (start 75.095 -91.955) (end 75.095 -89.145) (width 0.2) (layer F.Cu) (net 34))
 (segment (start 73.25 -93.8) (end 75.095 -91.955) (width 0.2) (layer F.Cu) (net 34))
 (segment (start 72.725 -93.8) (end 73.25 -93.8) (width 0.2) (layer F.Cu) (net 34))
 (segment (start 73.825 -92.3) (end 73.825 -89.145) (width 0.2) (layer F.Cu) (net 33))
 (segment (start 72.725 -93.4) (end 73.825 -92.3) (width 0.2) (layer F.Cu) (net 33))
 (segment (start 72.555 -89.695) (end 72.555 -89.145) (width 0.2) (layer F.Cu) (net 32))
 (segment (start 71.1 -91.15) (end 72.555 -89.695) (width 0.2) (layer F.Cu) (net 32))
 (segment (start 71.1 -92.575) (end 71.1 -91.15) (width 0.2) (layer F.Cu) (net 32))
 (segment (start 70.74759 -89.68241) (end 71.285 -89.145) (width 0.2) (layer F.Cu) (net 31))
 (segment (start 70.7 -92.396766) (end 70.74759 -92.349176) (width 0.2) (layer F.Cu) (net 31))
 (segment (start 70.74759 -92.349176) (end 70.74759 -89.68241) (width 0.2) (layer F.Cu) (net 31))
 (segment (start 70.7 -92.575) (end 70.7 -92.396766) (width 0.2) (layer F.Cu) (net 31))
 (segment (start 70.36202 -92.236363) (end 70.36202 -90.56202) (width 0.2) (layer F.Cu) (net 30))
 (segment (start 70.3 -92.298383) (end 70.36202 -92.236363) (width 0.2) (layer F.Cu) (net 30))
 (segment (start 70.3 -92.575) (end 70.3 -92.298383) (width 0.2) (layer F.Cu) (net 30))
 (segment (start 70.015 -90.215) (end 70.015 -89.145) (width 0.2) (layer F.Cu) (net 30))
 (segment (start 70.36202 -90.56202) (end 70.015 -90.215) (width 0.2) (layer F.Cu) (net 30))
 (segment (start 70.009611 -90.959611) (end 68.745 -89.695) (width 0.2) (layer F.Cu) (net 29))
 (segment (start 68.745 -89.695) (end 68.745 -89.145) (width 0.2) (layer F.Cu) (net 29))
 (segment (start 70.00961 -92.09039) (end 70.009611 -90.959611) (width 0.2) (layer F.Cu) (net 29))
 (segment (start 69.9 -92.2) (end 70.00961 -92.09039) (width 0.2) (layer F.Cu) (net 29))
 (segment (start 69.9 -92.575) (end 69.9 -92.2) (width 0.2) (layer F.Cu) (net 29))
 (segment (start 69.557201 -91.867457) (end 69.5 -91.924658) (width 0.2) (layer F.Cu) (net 28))
 (segment (start 69.557201 -91.332543) (end 69.557201 -91.867457) (width 0.2) (layer F.Cu) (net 28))
 (segment (start 69.124658 -90.9) (end 69.557201 -91.332543) (width 0.2) (layer F.Cu) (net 28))
 (segment (start 68.52304 -90.9) (end 69.124658 -90.9) (width 0.2) (layer F.Cu) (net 28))
 (segment (start 67.475 -89.85196) (end 68.52304 -90.9) (width 0.2) (layer F.Cu) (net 28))
 (segment (start 69.5 -91.924658) (end 69.5 -92.575) (width 0.2) (layer F.Cu) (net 28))
 (segment (start 67.475 -89.145) (end 67.475 -89.85196) (width 0.2) (layer F.Cu) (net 28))
 (segment (start 69.1 -91.7) (end 69 -91.6) (width 0.2) (layer F.Cu) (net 38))
 (segment (start 69.1 -92.575) (end 69.1 -91.7) (width 0.2) (layer F.Cu) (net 38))
 (segment (start 66.205 -89.695) (end 66.205 -89.145) (width 0.2) (layer F.Cu) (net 27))
 (segment (start 67.967457 -90.842799) (end 67.352799 -90.842799) (width 0.2) (layer F.Cu) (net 27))
 (segment (start 68.257201 -91.132543) (end 67.967457 -90.842799) (width 0.2) (layer F.Cu) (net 27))
 (segment (start 67.352799 -90.842799) (end 66.205 -89.695) (width 0.2) (layer F.Cu) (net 27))
 (segment (start 68.7 -92.575) (end 68.7 -92.251617) (width 0.2) (layer F.Cu) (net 27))
 (segment (start 68.462799 -91.237201) (end 68.46759 -91.23241) (width 0.16) (layer F.Cu) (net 27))
 (segment (start 68.462799 -91.857857) (end 68.462799 -91.237201) (width 0.16) (layer F.Cu) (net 27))
 (segment (start 68.7 -92.095058) (end 68.462799 -91.857857) (width 0.16) (layer F.Cu) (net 27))
 (segment (start 68.7 -92.575) (end 68.7 -92.095058) (width 0.16) (layer F.Cu) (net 27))
 (segment (start 68.357068 -91.23241) (end 68.257201 -91.132543) (width 0.16) (layer F.Cu) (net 27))
 (segment (start 68.46759 -91.23241) (end 68.357068 -91.23241) (width 0.16) (layer F.Cu) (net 27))
 (segment (start 67.7 -91.581519) (end 68.3 -92.181519) (width 0.16) (layer F.Cu) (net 39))
 (segment (start 68.3 -92.181519) (end 68.3 -92.575) (width 0.16) (layer F.Cu) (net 39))
 (segment (start 67.7 -91.4) (end 67.7 -91.581519) (width 0.16) (layer F.Cu) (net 39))
 (segment (start 62.402401 -90.397401) (end 65.945784 -90.397401) (width 0.2) (layer F.Cu) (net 26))
 (segment (start 62.15 -90.145) (end 62.402401 -90.397401) (width 0.2) (layer F.Cu) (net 26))
 (segment (start 67.9 -92.251617) (end 67.624192 -91.975809) (width 0.2) (layer F.Cu) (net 26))
 (segment (start 67.9 -92.575) (end 67.9 -92.251617) (width 0.2) (layer F.Cu) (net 26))
 (segment (start 65.945784 -90.470442) (end 65.945784 -90.397401) (width 0.2) (layer F.Cu) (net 26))
 (segment (start 67.451151 -91.975809) (end 65.945784 -90.470442) (width 0.2) (layer F.Cu) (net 26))
 (segment (start 67.624192 -91.975809) (end 67.451151 -91.975809) (width 0.2) (layer F.Cu) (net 26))
 (segment (start 63.390046 -91.415) (end 62.15 -91.415) (width 0.2) (layer F.Cu) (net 25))
 (segment (start 65.775046 -93.8) (end 63.390046 -91.415) (width 0.2) (layer F.Cu) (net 25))
 (segment (start 66.575 -93.8) (end 65.775046 -93.8) (width 0.2) (layer F.Cu) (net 25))
 (segment (start 66.575 -94.2) (end 65.676664 -94.2) (width 0.2) (layer F.Cu) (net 24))
 (segment (start 64.161664 -92.685) (end 62.15 -92.685) (width 0.2) (layer F.Cu) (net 24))
 (segment (start 65.676664 -94.2) (end 64.161664 -92.685) (width 0.2) (layer F.Cu) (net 24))
 (segment (start 66.575 -94.6) (end 65.578282 -94.6) (width 0.2) (layer F.Cu) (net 23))
 (segment (start 64.933282 -93.955) (end 62.15 -93.955) (width 0.2) (layer F.Cu) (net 23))
 (segment (start 65.578282 -94.6) (end 64.933282 -93.955) (width 0.2) (layer F.Cu) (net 23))
 (segment (start 62.375 -95) (end 62.15 -95.225) (width 0.2) (layer F.Cu) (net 22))
 (segment (start 66.575 -95) (end 62.375 -95) (width 0.2) (layer F.Cu) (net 22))
 (segment (start 66.575 -95.4) (end 63.84759 -95.4) (width 0.2) (layer F.Cu) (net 21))
 (segment (start 62.784322 -96.495) (end 62.15 -96.495) (width 0.2) (layer F.Cu) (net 21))
 (segment (start 63.84759 -95.431732) (end 62.784322 -96.495) (width 0.2) (layer F.Cu) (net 21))
 (segment (start 63.84759 -95.4) (end 63.84759 -95.431732) (width 0.2) (layer F.Cu) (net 21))
 (segment (start 66.575 -95.8) (end 65.6 -95.8) (width 0.2) (layer F.Cu) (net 20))
 (segment (start 63.635 -97.765) (end 62.15 -97.765) (width 0.2) (layer F.Cu) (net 20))
 (segment (start 65.6 -95.8) (end 63.635 -97.765) (width 0.2) (layer F.Cu) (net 20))
 (segment (start 66.575 -96.2) (end 65.8 -96.2) (width 0.2) (layer F.Cu) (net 19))
 (segment (start 62.965 -99.035) (end 62.15 -99.035) (width 0.2) (layer F.Cu) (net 19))
 (segment (start 65.8 -96.2) (end 62.965 -99.035) (width 0.2) (layer F.Cu) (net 19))
 (segment (start 66.05 -96.6) (end 63.5 -99.15) (width 0.2) (layer F.Cu) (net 18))
 (segment (start 66.575 -96.6) (end 66.05 -96.6) (width 0.2) (layer F.Cu) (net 18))
 (segment (start 63.35 -100.305) (end 62.15 -100.305) (width 0.2) (layer F.Cu) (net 18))
 (segment (start 63.5 -100.155) (end 63.35 -100.305) (width 0.2) (layer F.Cu) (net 18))
 (segment (start 63.5 -99.15) (end 63.5 -100.155) (width 0.2) (layer F.Cu) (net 18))
 (segment (start 62.784322 -101.575) (end 62.15 -101.575) (width 0.2) (layer F.Cu) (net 17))
 (segment (start 63.85241 -100.506912) (end 62.784322 -101.575) (width 0.2) (layer F.Cu) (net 17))
 (segment (start 63.85241 -99.399207) (end 63.85241 -100.506912) (width 0.2) (layer F.Cu) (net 17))
 (segment (start 66.251617 -97) (end 63.85241 -99.399207) (width 0.2) (layer F.Cu) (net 17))
 (segment (start 66.575 -97) (end 66.251617 -97) (width 0.2) (layer F.Cu) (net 17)))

